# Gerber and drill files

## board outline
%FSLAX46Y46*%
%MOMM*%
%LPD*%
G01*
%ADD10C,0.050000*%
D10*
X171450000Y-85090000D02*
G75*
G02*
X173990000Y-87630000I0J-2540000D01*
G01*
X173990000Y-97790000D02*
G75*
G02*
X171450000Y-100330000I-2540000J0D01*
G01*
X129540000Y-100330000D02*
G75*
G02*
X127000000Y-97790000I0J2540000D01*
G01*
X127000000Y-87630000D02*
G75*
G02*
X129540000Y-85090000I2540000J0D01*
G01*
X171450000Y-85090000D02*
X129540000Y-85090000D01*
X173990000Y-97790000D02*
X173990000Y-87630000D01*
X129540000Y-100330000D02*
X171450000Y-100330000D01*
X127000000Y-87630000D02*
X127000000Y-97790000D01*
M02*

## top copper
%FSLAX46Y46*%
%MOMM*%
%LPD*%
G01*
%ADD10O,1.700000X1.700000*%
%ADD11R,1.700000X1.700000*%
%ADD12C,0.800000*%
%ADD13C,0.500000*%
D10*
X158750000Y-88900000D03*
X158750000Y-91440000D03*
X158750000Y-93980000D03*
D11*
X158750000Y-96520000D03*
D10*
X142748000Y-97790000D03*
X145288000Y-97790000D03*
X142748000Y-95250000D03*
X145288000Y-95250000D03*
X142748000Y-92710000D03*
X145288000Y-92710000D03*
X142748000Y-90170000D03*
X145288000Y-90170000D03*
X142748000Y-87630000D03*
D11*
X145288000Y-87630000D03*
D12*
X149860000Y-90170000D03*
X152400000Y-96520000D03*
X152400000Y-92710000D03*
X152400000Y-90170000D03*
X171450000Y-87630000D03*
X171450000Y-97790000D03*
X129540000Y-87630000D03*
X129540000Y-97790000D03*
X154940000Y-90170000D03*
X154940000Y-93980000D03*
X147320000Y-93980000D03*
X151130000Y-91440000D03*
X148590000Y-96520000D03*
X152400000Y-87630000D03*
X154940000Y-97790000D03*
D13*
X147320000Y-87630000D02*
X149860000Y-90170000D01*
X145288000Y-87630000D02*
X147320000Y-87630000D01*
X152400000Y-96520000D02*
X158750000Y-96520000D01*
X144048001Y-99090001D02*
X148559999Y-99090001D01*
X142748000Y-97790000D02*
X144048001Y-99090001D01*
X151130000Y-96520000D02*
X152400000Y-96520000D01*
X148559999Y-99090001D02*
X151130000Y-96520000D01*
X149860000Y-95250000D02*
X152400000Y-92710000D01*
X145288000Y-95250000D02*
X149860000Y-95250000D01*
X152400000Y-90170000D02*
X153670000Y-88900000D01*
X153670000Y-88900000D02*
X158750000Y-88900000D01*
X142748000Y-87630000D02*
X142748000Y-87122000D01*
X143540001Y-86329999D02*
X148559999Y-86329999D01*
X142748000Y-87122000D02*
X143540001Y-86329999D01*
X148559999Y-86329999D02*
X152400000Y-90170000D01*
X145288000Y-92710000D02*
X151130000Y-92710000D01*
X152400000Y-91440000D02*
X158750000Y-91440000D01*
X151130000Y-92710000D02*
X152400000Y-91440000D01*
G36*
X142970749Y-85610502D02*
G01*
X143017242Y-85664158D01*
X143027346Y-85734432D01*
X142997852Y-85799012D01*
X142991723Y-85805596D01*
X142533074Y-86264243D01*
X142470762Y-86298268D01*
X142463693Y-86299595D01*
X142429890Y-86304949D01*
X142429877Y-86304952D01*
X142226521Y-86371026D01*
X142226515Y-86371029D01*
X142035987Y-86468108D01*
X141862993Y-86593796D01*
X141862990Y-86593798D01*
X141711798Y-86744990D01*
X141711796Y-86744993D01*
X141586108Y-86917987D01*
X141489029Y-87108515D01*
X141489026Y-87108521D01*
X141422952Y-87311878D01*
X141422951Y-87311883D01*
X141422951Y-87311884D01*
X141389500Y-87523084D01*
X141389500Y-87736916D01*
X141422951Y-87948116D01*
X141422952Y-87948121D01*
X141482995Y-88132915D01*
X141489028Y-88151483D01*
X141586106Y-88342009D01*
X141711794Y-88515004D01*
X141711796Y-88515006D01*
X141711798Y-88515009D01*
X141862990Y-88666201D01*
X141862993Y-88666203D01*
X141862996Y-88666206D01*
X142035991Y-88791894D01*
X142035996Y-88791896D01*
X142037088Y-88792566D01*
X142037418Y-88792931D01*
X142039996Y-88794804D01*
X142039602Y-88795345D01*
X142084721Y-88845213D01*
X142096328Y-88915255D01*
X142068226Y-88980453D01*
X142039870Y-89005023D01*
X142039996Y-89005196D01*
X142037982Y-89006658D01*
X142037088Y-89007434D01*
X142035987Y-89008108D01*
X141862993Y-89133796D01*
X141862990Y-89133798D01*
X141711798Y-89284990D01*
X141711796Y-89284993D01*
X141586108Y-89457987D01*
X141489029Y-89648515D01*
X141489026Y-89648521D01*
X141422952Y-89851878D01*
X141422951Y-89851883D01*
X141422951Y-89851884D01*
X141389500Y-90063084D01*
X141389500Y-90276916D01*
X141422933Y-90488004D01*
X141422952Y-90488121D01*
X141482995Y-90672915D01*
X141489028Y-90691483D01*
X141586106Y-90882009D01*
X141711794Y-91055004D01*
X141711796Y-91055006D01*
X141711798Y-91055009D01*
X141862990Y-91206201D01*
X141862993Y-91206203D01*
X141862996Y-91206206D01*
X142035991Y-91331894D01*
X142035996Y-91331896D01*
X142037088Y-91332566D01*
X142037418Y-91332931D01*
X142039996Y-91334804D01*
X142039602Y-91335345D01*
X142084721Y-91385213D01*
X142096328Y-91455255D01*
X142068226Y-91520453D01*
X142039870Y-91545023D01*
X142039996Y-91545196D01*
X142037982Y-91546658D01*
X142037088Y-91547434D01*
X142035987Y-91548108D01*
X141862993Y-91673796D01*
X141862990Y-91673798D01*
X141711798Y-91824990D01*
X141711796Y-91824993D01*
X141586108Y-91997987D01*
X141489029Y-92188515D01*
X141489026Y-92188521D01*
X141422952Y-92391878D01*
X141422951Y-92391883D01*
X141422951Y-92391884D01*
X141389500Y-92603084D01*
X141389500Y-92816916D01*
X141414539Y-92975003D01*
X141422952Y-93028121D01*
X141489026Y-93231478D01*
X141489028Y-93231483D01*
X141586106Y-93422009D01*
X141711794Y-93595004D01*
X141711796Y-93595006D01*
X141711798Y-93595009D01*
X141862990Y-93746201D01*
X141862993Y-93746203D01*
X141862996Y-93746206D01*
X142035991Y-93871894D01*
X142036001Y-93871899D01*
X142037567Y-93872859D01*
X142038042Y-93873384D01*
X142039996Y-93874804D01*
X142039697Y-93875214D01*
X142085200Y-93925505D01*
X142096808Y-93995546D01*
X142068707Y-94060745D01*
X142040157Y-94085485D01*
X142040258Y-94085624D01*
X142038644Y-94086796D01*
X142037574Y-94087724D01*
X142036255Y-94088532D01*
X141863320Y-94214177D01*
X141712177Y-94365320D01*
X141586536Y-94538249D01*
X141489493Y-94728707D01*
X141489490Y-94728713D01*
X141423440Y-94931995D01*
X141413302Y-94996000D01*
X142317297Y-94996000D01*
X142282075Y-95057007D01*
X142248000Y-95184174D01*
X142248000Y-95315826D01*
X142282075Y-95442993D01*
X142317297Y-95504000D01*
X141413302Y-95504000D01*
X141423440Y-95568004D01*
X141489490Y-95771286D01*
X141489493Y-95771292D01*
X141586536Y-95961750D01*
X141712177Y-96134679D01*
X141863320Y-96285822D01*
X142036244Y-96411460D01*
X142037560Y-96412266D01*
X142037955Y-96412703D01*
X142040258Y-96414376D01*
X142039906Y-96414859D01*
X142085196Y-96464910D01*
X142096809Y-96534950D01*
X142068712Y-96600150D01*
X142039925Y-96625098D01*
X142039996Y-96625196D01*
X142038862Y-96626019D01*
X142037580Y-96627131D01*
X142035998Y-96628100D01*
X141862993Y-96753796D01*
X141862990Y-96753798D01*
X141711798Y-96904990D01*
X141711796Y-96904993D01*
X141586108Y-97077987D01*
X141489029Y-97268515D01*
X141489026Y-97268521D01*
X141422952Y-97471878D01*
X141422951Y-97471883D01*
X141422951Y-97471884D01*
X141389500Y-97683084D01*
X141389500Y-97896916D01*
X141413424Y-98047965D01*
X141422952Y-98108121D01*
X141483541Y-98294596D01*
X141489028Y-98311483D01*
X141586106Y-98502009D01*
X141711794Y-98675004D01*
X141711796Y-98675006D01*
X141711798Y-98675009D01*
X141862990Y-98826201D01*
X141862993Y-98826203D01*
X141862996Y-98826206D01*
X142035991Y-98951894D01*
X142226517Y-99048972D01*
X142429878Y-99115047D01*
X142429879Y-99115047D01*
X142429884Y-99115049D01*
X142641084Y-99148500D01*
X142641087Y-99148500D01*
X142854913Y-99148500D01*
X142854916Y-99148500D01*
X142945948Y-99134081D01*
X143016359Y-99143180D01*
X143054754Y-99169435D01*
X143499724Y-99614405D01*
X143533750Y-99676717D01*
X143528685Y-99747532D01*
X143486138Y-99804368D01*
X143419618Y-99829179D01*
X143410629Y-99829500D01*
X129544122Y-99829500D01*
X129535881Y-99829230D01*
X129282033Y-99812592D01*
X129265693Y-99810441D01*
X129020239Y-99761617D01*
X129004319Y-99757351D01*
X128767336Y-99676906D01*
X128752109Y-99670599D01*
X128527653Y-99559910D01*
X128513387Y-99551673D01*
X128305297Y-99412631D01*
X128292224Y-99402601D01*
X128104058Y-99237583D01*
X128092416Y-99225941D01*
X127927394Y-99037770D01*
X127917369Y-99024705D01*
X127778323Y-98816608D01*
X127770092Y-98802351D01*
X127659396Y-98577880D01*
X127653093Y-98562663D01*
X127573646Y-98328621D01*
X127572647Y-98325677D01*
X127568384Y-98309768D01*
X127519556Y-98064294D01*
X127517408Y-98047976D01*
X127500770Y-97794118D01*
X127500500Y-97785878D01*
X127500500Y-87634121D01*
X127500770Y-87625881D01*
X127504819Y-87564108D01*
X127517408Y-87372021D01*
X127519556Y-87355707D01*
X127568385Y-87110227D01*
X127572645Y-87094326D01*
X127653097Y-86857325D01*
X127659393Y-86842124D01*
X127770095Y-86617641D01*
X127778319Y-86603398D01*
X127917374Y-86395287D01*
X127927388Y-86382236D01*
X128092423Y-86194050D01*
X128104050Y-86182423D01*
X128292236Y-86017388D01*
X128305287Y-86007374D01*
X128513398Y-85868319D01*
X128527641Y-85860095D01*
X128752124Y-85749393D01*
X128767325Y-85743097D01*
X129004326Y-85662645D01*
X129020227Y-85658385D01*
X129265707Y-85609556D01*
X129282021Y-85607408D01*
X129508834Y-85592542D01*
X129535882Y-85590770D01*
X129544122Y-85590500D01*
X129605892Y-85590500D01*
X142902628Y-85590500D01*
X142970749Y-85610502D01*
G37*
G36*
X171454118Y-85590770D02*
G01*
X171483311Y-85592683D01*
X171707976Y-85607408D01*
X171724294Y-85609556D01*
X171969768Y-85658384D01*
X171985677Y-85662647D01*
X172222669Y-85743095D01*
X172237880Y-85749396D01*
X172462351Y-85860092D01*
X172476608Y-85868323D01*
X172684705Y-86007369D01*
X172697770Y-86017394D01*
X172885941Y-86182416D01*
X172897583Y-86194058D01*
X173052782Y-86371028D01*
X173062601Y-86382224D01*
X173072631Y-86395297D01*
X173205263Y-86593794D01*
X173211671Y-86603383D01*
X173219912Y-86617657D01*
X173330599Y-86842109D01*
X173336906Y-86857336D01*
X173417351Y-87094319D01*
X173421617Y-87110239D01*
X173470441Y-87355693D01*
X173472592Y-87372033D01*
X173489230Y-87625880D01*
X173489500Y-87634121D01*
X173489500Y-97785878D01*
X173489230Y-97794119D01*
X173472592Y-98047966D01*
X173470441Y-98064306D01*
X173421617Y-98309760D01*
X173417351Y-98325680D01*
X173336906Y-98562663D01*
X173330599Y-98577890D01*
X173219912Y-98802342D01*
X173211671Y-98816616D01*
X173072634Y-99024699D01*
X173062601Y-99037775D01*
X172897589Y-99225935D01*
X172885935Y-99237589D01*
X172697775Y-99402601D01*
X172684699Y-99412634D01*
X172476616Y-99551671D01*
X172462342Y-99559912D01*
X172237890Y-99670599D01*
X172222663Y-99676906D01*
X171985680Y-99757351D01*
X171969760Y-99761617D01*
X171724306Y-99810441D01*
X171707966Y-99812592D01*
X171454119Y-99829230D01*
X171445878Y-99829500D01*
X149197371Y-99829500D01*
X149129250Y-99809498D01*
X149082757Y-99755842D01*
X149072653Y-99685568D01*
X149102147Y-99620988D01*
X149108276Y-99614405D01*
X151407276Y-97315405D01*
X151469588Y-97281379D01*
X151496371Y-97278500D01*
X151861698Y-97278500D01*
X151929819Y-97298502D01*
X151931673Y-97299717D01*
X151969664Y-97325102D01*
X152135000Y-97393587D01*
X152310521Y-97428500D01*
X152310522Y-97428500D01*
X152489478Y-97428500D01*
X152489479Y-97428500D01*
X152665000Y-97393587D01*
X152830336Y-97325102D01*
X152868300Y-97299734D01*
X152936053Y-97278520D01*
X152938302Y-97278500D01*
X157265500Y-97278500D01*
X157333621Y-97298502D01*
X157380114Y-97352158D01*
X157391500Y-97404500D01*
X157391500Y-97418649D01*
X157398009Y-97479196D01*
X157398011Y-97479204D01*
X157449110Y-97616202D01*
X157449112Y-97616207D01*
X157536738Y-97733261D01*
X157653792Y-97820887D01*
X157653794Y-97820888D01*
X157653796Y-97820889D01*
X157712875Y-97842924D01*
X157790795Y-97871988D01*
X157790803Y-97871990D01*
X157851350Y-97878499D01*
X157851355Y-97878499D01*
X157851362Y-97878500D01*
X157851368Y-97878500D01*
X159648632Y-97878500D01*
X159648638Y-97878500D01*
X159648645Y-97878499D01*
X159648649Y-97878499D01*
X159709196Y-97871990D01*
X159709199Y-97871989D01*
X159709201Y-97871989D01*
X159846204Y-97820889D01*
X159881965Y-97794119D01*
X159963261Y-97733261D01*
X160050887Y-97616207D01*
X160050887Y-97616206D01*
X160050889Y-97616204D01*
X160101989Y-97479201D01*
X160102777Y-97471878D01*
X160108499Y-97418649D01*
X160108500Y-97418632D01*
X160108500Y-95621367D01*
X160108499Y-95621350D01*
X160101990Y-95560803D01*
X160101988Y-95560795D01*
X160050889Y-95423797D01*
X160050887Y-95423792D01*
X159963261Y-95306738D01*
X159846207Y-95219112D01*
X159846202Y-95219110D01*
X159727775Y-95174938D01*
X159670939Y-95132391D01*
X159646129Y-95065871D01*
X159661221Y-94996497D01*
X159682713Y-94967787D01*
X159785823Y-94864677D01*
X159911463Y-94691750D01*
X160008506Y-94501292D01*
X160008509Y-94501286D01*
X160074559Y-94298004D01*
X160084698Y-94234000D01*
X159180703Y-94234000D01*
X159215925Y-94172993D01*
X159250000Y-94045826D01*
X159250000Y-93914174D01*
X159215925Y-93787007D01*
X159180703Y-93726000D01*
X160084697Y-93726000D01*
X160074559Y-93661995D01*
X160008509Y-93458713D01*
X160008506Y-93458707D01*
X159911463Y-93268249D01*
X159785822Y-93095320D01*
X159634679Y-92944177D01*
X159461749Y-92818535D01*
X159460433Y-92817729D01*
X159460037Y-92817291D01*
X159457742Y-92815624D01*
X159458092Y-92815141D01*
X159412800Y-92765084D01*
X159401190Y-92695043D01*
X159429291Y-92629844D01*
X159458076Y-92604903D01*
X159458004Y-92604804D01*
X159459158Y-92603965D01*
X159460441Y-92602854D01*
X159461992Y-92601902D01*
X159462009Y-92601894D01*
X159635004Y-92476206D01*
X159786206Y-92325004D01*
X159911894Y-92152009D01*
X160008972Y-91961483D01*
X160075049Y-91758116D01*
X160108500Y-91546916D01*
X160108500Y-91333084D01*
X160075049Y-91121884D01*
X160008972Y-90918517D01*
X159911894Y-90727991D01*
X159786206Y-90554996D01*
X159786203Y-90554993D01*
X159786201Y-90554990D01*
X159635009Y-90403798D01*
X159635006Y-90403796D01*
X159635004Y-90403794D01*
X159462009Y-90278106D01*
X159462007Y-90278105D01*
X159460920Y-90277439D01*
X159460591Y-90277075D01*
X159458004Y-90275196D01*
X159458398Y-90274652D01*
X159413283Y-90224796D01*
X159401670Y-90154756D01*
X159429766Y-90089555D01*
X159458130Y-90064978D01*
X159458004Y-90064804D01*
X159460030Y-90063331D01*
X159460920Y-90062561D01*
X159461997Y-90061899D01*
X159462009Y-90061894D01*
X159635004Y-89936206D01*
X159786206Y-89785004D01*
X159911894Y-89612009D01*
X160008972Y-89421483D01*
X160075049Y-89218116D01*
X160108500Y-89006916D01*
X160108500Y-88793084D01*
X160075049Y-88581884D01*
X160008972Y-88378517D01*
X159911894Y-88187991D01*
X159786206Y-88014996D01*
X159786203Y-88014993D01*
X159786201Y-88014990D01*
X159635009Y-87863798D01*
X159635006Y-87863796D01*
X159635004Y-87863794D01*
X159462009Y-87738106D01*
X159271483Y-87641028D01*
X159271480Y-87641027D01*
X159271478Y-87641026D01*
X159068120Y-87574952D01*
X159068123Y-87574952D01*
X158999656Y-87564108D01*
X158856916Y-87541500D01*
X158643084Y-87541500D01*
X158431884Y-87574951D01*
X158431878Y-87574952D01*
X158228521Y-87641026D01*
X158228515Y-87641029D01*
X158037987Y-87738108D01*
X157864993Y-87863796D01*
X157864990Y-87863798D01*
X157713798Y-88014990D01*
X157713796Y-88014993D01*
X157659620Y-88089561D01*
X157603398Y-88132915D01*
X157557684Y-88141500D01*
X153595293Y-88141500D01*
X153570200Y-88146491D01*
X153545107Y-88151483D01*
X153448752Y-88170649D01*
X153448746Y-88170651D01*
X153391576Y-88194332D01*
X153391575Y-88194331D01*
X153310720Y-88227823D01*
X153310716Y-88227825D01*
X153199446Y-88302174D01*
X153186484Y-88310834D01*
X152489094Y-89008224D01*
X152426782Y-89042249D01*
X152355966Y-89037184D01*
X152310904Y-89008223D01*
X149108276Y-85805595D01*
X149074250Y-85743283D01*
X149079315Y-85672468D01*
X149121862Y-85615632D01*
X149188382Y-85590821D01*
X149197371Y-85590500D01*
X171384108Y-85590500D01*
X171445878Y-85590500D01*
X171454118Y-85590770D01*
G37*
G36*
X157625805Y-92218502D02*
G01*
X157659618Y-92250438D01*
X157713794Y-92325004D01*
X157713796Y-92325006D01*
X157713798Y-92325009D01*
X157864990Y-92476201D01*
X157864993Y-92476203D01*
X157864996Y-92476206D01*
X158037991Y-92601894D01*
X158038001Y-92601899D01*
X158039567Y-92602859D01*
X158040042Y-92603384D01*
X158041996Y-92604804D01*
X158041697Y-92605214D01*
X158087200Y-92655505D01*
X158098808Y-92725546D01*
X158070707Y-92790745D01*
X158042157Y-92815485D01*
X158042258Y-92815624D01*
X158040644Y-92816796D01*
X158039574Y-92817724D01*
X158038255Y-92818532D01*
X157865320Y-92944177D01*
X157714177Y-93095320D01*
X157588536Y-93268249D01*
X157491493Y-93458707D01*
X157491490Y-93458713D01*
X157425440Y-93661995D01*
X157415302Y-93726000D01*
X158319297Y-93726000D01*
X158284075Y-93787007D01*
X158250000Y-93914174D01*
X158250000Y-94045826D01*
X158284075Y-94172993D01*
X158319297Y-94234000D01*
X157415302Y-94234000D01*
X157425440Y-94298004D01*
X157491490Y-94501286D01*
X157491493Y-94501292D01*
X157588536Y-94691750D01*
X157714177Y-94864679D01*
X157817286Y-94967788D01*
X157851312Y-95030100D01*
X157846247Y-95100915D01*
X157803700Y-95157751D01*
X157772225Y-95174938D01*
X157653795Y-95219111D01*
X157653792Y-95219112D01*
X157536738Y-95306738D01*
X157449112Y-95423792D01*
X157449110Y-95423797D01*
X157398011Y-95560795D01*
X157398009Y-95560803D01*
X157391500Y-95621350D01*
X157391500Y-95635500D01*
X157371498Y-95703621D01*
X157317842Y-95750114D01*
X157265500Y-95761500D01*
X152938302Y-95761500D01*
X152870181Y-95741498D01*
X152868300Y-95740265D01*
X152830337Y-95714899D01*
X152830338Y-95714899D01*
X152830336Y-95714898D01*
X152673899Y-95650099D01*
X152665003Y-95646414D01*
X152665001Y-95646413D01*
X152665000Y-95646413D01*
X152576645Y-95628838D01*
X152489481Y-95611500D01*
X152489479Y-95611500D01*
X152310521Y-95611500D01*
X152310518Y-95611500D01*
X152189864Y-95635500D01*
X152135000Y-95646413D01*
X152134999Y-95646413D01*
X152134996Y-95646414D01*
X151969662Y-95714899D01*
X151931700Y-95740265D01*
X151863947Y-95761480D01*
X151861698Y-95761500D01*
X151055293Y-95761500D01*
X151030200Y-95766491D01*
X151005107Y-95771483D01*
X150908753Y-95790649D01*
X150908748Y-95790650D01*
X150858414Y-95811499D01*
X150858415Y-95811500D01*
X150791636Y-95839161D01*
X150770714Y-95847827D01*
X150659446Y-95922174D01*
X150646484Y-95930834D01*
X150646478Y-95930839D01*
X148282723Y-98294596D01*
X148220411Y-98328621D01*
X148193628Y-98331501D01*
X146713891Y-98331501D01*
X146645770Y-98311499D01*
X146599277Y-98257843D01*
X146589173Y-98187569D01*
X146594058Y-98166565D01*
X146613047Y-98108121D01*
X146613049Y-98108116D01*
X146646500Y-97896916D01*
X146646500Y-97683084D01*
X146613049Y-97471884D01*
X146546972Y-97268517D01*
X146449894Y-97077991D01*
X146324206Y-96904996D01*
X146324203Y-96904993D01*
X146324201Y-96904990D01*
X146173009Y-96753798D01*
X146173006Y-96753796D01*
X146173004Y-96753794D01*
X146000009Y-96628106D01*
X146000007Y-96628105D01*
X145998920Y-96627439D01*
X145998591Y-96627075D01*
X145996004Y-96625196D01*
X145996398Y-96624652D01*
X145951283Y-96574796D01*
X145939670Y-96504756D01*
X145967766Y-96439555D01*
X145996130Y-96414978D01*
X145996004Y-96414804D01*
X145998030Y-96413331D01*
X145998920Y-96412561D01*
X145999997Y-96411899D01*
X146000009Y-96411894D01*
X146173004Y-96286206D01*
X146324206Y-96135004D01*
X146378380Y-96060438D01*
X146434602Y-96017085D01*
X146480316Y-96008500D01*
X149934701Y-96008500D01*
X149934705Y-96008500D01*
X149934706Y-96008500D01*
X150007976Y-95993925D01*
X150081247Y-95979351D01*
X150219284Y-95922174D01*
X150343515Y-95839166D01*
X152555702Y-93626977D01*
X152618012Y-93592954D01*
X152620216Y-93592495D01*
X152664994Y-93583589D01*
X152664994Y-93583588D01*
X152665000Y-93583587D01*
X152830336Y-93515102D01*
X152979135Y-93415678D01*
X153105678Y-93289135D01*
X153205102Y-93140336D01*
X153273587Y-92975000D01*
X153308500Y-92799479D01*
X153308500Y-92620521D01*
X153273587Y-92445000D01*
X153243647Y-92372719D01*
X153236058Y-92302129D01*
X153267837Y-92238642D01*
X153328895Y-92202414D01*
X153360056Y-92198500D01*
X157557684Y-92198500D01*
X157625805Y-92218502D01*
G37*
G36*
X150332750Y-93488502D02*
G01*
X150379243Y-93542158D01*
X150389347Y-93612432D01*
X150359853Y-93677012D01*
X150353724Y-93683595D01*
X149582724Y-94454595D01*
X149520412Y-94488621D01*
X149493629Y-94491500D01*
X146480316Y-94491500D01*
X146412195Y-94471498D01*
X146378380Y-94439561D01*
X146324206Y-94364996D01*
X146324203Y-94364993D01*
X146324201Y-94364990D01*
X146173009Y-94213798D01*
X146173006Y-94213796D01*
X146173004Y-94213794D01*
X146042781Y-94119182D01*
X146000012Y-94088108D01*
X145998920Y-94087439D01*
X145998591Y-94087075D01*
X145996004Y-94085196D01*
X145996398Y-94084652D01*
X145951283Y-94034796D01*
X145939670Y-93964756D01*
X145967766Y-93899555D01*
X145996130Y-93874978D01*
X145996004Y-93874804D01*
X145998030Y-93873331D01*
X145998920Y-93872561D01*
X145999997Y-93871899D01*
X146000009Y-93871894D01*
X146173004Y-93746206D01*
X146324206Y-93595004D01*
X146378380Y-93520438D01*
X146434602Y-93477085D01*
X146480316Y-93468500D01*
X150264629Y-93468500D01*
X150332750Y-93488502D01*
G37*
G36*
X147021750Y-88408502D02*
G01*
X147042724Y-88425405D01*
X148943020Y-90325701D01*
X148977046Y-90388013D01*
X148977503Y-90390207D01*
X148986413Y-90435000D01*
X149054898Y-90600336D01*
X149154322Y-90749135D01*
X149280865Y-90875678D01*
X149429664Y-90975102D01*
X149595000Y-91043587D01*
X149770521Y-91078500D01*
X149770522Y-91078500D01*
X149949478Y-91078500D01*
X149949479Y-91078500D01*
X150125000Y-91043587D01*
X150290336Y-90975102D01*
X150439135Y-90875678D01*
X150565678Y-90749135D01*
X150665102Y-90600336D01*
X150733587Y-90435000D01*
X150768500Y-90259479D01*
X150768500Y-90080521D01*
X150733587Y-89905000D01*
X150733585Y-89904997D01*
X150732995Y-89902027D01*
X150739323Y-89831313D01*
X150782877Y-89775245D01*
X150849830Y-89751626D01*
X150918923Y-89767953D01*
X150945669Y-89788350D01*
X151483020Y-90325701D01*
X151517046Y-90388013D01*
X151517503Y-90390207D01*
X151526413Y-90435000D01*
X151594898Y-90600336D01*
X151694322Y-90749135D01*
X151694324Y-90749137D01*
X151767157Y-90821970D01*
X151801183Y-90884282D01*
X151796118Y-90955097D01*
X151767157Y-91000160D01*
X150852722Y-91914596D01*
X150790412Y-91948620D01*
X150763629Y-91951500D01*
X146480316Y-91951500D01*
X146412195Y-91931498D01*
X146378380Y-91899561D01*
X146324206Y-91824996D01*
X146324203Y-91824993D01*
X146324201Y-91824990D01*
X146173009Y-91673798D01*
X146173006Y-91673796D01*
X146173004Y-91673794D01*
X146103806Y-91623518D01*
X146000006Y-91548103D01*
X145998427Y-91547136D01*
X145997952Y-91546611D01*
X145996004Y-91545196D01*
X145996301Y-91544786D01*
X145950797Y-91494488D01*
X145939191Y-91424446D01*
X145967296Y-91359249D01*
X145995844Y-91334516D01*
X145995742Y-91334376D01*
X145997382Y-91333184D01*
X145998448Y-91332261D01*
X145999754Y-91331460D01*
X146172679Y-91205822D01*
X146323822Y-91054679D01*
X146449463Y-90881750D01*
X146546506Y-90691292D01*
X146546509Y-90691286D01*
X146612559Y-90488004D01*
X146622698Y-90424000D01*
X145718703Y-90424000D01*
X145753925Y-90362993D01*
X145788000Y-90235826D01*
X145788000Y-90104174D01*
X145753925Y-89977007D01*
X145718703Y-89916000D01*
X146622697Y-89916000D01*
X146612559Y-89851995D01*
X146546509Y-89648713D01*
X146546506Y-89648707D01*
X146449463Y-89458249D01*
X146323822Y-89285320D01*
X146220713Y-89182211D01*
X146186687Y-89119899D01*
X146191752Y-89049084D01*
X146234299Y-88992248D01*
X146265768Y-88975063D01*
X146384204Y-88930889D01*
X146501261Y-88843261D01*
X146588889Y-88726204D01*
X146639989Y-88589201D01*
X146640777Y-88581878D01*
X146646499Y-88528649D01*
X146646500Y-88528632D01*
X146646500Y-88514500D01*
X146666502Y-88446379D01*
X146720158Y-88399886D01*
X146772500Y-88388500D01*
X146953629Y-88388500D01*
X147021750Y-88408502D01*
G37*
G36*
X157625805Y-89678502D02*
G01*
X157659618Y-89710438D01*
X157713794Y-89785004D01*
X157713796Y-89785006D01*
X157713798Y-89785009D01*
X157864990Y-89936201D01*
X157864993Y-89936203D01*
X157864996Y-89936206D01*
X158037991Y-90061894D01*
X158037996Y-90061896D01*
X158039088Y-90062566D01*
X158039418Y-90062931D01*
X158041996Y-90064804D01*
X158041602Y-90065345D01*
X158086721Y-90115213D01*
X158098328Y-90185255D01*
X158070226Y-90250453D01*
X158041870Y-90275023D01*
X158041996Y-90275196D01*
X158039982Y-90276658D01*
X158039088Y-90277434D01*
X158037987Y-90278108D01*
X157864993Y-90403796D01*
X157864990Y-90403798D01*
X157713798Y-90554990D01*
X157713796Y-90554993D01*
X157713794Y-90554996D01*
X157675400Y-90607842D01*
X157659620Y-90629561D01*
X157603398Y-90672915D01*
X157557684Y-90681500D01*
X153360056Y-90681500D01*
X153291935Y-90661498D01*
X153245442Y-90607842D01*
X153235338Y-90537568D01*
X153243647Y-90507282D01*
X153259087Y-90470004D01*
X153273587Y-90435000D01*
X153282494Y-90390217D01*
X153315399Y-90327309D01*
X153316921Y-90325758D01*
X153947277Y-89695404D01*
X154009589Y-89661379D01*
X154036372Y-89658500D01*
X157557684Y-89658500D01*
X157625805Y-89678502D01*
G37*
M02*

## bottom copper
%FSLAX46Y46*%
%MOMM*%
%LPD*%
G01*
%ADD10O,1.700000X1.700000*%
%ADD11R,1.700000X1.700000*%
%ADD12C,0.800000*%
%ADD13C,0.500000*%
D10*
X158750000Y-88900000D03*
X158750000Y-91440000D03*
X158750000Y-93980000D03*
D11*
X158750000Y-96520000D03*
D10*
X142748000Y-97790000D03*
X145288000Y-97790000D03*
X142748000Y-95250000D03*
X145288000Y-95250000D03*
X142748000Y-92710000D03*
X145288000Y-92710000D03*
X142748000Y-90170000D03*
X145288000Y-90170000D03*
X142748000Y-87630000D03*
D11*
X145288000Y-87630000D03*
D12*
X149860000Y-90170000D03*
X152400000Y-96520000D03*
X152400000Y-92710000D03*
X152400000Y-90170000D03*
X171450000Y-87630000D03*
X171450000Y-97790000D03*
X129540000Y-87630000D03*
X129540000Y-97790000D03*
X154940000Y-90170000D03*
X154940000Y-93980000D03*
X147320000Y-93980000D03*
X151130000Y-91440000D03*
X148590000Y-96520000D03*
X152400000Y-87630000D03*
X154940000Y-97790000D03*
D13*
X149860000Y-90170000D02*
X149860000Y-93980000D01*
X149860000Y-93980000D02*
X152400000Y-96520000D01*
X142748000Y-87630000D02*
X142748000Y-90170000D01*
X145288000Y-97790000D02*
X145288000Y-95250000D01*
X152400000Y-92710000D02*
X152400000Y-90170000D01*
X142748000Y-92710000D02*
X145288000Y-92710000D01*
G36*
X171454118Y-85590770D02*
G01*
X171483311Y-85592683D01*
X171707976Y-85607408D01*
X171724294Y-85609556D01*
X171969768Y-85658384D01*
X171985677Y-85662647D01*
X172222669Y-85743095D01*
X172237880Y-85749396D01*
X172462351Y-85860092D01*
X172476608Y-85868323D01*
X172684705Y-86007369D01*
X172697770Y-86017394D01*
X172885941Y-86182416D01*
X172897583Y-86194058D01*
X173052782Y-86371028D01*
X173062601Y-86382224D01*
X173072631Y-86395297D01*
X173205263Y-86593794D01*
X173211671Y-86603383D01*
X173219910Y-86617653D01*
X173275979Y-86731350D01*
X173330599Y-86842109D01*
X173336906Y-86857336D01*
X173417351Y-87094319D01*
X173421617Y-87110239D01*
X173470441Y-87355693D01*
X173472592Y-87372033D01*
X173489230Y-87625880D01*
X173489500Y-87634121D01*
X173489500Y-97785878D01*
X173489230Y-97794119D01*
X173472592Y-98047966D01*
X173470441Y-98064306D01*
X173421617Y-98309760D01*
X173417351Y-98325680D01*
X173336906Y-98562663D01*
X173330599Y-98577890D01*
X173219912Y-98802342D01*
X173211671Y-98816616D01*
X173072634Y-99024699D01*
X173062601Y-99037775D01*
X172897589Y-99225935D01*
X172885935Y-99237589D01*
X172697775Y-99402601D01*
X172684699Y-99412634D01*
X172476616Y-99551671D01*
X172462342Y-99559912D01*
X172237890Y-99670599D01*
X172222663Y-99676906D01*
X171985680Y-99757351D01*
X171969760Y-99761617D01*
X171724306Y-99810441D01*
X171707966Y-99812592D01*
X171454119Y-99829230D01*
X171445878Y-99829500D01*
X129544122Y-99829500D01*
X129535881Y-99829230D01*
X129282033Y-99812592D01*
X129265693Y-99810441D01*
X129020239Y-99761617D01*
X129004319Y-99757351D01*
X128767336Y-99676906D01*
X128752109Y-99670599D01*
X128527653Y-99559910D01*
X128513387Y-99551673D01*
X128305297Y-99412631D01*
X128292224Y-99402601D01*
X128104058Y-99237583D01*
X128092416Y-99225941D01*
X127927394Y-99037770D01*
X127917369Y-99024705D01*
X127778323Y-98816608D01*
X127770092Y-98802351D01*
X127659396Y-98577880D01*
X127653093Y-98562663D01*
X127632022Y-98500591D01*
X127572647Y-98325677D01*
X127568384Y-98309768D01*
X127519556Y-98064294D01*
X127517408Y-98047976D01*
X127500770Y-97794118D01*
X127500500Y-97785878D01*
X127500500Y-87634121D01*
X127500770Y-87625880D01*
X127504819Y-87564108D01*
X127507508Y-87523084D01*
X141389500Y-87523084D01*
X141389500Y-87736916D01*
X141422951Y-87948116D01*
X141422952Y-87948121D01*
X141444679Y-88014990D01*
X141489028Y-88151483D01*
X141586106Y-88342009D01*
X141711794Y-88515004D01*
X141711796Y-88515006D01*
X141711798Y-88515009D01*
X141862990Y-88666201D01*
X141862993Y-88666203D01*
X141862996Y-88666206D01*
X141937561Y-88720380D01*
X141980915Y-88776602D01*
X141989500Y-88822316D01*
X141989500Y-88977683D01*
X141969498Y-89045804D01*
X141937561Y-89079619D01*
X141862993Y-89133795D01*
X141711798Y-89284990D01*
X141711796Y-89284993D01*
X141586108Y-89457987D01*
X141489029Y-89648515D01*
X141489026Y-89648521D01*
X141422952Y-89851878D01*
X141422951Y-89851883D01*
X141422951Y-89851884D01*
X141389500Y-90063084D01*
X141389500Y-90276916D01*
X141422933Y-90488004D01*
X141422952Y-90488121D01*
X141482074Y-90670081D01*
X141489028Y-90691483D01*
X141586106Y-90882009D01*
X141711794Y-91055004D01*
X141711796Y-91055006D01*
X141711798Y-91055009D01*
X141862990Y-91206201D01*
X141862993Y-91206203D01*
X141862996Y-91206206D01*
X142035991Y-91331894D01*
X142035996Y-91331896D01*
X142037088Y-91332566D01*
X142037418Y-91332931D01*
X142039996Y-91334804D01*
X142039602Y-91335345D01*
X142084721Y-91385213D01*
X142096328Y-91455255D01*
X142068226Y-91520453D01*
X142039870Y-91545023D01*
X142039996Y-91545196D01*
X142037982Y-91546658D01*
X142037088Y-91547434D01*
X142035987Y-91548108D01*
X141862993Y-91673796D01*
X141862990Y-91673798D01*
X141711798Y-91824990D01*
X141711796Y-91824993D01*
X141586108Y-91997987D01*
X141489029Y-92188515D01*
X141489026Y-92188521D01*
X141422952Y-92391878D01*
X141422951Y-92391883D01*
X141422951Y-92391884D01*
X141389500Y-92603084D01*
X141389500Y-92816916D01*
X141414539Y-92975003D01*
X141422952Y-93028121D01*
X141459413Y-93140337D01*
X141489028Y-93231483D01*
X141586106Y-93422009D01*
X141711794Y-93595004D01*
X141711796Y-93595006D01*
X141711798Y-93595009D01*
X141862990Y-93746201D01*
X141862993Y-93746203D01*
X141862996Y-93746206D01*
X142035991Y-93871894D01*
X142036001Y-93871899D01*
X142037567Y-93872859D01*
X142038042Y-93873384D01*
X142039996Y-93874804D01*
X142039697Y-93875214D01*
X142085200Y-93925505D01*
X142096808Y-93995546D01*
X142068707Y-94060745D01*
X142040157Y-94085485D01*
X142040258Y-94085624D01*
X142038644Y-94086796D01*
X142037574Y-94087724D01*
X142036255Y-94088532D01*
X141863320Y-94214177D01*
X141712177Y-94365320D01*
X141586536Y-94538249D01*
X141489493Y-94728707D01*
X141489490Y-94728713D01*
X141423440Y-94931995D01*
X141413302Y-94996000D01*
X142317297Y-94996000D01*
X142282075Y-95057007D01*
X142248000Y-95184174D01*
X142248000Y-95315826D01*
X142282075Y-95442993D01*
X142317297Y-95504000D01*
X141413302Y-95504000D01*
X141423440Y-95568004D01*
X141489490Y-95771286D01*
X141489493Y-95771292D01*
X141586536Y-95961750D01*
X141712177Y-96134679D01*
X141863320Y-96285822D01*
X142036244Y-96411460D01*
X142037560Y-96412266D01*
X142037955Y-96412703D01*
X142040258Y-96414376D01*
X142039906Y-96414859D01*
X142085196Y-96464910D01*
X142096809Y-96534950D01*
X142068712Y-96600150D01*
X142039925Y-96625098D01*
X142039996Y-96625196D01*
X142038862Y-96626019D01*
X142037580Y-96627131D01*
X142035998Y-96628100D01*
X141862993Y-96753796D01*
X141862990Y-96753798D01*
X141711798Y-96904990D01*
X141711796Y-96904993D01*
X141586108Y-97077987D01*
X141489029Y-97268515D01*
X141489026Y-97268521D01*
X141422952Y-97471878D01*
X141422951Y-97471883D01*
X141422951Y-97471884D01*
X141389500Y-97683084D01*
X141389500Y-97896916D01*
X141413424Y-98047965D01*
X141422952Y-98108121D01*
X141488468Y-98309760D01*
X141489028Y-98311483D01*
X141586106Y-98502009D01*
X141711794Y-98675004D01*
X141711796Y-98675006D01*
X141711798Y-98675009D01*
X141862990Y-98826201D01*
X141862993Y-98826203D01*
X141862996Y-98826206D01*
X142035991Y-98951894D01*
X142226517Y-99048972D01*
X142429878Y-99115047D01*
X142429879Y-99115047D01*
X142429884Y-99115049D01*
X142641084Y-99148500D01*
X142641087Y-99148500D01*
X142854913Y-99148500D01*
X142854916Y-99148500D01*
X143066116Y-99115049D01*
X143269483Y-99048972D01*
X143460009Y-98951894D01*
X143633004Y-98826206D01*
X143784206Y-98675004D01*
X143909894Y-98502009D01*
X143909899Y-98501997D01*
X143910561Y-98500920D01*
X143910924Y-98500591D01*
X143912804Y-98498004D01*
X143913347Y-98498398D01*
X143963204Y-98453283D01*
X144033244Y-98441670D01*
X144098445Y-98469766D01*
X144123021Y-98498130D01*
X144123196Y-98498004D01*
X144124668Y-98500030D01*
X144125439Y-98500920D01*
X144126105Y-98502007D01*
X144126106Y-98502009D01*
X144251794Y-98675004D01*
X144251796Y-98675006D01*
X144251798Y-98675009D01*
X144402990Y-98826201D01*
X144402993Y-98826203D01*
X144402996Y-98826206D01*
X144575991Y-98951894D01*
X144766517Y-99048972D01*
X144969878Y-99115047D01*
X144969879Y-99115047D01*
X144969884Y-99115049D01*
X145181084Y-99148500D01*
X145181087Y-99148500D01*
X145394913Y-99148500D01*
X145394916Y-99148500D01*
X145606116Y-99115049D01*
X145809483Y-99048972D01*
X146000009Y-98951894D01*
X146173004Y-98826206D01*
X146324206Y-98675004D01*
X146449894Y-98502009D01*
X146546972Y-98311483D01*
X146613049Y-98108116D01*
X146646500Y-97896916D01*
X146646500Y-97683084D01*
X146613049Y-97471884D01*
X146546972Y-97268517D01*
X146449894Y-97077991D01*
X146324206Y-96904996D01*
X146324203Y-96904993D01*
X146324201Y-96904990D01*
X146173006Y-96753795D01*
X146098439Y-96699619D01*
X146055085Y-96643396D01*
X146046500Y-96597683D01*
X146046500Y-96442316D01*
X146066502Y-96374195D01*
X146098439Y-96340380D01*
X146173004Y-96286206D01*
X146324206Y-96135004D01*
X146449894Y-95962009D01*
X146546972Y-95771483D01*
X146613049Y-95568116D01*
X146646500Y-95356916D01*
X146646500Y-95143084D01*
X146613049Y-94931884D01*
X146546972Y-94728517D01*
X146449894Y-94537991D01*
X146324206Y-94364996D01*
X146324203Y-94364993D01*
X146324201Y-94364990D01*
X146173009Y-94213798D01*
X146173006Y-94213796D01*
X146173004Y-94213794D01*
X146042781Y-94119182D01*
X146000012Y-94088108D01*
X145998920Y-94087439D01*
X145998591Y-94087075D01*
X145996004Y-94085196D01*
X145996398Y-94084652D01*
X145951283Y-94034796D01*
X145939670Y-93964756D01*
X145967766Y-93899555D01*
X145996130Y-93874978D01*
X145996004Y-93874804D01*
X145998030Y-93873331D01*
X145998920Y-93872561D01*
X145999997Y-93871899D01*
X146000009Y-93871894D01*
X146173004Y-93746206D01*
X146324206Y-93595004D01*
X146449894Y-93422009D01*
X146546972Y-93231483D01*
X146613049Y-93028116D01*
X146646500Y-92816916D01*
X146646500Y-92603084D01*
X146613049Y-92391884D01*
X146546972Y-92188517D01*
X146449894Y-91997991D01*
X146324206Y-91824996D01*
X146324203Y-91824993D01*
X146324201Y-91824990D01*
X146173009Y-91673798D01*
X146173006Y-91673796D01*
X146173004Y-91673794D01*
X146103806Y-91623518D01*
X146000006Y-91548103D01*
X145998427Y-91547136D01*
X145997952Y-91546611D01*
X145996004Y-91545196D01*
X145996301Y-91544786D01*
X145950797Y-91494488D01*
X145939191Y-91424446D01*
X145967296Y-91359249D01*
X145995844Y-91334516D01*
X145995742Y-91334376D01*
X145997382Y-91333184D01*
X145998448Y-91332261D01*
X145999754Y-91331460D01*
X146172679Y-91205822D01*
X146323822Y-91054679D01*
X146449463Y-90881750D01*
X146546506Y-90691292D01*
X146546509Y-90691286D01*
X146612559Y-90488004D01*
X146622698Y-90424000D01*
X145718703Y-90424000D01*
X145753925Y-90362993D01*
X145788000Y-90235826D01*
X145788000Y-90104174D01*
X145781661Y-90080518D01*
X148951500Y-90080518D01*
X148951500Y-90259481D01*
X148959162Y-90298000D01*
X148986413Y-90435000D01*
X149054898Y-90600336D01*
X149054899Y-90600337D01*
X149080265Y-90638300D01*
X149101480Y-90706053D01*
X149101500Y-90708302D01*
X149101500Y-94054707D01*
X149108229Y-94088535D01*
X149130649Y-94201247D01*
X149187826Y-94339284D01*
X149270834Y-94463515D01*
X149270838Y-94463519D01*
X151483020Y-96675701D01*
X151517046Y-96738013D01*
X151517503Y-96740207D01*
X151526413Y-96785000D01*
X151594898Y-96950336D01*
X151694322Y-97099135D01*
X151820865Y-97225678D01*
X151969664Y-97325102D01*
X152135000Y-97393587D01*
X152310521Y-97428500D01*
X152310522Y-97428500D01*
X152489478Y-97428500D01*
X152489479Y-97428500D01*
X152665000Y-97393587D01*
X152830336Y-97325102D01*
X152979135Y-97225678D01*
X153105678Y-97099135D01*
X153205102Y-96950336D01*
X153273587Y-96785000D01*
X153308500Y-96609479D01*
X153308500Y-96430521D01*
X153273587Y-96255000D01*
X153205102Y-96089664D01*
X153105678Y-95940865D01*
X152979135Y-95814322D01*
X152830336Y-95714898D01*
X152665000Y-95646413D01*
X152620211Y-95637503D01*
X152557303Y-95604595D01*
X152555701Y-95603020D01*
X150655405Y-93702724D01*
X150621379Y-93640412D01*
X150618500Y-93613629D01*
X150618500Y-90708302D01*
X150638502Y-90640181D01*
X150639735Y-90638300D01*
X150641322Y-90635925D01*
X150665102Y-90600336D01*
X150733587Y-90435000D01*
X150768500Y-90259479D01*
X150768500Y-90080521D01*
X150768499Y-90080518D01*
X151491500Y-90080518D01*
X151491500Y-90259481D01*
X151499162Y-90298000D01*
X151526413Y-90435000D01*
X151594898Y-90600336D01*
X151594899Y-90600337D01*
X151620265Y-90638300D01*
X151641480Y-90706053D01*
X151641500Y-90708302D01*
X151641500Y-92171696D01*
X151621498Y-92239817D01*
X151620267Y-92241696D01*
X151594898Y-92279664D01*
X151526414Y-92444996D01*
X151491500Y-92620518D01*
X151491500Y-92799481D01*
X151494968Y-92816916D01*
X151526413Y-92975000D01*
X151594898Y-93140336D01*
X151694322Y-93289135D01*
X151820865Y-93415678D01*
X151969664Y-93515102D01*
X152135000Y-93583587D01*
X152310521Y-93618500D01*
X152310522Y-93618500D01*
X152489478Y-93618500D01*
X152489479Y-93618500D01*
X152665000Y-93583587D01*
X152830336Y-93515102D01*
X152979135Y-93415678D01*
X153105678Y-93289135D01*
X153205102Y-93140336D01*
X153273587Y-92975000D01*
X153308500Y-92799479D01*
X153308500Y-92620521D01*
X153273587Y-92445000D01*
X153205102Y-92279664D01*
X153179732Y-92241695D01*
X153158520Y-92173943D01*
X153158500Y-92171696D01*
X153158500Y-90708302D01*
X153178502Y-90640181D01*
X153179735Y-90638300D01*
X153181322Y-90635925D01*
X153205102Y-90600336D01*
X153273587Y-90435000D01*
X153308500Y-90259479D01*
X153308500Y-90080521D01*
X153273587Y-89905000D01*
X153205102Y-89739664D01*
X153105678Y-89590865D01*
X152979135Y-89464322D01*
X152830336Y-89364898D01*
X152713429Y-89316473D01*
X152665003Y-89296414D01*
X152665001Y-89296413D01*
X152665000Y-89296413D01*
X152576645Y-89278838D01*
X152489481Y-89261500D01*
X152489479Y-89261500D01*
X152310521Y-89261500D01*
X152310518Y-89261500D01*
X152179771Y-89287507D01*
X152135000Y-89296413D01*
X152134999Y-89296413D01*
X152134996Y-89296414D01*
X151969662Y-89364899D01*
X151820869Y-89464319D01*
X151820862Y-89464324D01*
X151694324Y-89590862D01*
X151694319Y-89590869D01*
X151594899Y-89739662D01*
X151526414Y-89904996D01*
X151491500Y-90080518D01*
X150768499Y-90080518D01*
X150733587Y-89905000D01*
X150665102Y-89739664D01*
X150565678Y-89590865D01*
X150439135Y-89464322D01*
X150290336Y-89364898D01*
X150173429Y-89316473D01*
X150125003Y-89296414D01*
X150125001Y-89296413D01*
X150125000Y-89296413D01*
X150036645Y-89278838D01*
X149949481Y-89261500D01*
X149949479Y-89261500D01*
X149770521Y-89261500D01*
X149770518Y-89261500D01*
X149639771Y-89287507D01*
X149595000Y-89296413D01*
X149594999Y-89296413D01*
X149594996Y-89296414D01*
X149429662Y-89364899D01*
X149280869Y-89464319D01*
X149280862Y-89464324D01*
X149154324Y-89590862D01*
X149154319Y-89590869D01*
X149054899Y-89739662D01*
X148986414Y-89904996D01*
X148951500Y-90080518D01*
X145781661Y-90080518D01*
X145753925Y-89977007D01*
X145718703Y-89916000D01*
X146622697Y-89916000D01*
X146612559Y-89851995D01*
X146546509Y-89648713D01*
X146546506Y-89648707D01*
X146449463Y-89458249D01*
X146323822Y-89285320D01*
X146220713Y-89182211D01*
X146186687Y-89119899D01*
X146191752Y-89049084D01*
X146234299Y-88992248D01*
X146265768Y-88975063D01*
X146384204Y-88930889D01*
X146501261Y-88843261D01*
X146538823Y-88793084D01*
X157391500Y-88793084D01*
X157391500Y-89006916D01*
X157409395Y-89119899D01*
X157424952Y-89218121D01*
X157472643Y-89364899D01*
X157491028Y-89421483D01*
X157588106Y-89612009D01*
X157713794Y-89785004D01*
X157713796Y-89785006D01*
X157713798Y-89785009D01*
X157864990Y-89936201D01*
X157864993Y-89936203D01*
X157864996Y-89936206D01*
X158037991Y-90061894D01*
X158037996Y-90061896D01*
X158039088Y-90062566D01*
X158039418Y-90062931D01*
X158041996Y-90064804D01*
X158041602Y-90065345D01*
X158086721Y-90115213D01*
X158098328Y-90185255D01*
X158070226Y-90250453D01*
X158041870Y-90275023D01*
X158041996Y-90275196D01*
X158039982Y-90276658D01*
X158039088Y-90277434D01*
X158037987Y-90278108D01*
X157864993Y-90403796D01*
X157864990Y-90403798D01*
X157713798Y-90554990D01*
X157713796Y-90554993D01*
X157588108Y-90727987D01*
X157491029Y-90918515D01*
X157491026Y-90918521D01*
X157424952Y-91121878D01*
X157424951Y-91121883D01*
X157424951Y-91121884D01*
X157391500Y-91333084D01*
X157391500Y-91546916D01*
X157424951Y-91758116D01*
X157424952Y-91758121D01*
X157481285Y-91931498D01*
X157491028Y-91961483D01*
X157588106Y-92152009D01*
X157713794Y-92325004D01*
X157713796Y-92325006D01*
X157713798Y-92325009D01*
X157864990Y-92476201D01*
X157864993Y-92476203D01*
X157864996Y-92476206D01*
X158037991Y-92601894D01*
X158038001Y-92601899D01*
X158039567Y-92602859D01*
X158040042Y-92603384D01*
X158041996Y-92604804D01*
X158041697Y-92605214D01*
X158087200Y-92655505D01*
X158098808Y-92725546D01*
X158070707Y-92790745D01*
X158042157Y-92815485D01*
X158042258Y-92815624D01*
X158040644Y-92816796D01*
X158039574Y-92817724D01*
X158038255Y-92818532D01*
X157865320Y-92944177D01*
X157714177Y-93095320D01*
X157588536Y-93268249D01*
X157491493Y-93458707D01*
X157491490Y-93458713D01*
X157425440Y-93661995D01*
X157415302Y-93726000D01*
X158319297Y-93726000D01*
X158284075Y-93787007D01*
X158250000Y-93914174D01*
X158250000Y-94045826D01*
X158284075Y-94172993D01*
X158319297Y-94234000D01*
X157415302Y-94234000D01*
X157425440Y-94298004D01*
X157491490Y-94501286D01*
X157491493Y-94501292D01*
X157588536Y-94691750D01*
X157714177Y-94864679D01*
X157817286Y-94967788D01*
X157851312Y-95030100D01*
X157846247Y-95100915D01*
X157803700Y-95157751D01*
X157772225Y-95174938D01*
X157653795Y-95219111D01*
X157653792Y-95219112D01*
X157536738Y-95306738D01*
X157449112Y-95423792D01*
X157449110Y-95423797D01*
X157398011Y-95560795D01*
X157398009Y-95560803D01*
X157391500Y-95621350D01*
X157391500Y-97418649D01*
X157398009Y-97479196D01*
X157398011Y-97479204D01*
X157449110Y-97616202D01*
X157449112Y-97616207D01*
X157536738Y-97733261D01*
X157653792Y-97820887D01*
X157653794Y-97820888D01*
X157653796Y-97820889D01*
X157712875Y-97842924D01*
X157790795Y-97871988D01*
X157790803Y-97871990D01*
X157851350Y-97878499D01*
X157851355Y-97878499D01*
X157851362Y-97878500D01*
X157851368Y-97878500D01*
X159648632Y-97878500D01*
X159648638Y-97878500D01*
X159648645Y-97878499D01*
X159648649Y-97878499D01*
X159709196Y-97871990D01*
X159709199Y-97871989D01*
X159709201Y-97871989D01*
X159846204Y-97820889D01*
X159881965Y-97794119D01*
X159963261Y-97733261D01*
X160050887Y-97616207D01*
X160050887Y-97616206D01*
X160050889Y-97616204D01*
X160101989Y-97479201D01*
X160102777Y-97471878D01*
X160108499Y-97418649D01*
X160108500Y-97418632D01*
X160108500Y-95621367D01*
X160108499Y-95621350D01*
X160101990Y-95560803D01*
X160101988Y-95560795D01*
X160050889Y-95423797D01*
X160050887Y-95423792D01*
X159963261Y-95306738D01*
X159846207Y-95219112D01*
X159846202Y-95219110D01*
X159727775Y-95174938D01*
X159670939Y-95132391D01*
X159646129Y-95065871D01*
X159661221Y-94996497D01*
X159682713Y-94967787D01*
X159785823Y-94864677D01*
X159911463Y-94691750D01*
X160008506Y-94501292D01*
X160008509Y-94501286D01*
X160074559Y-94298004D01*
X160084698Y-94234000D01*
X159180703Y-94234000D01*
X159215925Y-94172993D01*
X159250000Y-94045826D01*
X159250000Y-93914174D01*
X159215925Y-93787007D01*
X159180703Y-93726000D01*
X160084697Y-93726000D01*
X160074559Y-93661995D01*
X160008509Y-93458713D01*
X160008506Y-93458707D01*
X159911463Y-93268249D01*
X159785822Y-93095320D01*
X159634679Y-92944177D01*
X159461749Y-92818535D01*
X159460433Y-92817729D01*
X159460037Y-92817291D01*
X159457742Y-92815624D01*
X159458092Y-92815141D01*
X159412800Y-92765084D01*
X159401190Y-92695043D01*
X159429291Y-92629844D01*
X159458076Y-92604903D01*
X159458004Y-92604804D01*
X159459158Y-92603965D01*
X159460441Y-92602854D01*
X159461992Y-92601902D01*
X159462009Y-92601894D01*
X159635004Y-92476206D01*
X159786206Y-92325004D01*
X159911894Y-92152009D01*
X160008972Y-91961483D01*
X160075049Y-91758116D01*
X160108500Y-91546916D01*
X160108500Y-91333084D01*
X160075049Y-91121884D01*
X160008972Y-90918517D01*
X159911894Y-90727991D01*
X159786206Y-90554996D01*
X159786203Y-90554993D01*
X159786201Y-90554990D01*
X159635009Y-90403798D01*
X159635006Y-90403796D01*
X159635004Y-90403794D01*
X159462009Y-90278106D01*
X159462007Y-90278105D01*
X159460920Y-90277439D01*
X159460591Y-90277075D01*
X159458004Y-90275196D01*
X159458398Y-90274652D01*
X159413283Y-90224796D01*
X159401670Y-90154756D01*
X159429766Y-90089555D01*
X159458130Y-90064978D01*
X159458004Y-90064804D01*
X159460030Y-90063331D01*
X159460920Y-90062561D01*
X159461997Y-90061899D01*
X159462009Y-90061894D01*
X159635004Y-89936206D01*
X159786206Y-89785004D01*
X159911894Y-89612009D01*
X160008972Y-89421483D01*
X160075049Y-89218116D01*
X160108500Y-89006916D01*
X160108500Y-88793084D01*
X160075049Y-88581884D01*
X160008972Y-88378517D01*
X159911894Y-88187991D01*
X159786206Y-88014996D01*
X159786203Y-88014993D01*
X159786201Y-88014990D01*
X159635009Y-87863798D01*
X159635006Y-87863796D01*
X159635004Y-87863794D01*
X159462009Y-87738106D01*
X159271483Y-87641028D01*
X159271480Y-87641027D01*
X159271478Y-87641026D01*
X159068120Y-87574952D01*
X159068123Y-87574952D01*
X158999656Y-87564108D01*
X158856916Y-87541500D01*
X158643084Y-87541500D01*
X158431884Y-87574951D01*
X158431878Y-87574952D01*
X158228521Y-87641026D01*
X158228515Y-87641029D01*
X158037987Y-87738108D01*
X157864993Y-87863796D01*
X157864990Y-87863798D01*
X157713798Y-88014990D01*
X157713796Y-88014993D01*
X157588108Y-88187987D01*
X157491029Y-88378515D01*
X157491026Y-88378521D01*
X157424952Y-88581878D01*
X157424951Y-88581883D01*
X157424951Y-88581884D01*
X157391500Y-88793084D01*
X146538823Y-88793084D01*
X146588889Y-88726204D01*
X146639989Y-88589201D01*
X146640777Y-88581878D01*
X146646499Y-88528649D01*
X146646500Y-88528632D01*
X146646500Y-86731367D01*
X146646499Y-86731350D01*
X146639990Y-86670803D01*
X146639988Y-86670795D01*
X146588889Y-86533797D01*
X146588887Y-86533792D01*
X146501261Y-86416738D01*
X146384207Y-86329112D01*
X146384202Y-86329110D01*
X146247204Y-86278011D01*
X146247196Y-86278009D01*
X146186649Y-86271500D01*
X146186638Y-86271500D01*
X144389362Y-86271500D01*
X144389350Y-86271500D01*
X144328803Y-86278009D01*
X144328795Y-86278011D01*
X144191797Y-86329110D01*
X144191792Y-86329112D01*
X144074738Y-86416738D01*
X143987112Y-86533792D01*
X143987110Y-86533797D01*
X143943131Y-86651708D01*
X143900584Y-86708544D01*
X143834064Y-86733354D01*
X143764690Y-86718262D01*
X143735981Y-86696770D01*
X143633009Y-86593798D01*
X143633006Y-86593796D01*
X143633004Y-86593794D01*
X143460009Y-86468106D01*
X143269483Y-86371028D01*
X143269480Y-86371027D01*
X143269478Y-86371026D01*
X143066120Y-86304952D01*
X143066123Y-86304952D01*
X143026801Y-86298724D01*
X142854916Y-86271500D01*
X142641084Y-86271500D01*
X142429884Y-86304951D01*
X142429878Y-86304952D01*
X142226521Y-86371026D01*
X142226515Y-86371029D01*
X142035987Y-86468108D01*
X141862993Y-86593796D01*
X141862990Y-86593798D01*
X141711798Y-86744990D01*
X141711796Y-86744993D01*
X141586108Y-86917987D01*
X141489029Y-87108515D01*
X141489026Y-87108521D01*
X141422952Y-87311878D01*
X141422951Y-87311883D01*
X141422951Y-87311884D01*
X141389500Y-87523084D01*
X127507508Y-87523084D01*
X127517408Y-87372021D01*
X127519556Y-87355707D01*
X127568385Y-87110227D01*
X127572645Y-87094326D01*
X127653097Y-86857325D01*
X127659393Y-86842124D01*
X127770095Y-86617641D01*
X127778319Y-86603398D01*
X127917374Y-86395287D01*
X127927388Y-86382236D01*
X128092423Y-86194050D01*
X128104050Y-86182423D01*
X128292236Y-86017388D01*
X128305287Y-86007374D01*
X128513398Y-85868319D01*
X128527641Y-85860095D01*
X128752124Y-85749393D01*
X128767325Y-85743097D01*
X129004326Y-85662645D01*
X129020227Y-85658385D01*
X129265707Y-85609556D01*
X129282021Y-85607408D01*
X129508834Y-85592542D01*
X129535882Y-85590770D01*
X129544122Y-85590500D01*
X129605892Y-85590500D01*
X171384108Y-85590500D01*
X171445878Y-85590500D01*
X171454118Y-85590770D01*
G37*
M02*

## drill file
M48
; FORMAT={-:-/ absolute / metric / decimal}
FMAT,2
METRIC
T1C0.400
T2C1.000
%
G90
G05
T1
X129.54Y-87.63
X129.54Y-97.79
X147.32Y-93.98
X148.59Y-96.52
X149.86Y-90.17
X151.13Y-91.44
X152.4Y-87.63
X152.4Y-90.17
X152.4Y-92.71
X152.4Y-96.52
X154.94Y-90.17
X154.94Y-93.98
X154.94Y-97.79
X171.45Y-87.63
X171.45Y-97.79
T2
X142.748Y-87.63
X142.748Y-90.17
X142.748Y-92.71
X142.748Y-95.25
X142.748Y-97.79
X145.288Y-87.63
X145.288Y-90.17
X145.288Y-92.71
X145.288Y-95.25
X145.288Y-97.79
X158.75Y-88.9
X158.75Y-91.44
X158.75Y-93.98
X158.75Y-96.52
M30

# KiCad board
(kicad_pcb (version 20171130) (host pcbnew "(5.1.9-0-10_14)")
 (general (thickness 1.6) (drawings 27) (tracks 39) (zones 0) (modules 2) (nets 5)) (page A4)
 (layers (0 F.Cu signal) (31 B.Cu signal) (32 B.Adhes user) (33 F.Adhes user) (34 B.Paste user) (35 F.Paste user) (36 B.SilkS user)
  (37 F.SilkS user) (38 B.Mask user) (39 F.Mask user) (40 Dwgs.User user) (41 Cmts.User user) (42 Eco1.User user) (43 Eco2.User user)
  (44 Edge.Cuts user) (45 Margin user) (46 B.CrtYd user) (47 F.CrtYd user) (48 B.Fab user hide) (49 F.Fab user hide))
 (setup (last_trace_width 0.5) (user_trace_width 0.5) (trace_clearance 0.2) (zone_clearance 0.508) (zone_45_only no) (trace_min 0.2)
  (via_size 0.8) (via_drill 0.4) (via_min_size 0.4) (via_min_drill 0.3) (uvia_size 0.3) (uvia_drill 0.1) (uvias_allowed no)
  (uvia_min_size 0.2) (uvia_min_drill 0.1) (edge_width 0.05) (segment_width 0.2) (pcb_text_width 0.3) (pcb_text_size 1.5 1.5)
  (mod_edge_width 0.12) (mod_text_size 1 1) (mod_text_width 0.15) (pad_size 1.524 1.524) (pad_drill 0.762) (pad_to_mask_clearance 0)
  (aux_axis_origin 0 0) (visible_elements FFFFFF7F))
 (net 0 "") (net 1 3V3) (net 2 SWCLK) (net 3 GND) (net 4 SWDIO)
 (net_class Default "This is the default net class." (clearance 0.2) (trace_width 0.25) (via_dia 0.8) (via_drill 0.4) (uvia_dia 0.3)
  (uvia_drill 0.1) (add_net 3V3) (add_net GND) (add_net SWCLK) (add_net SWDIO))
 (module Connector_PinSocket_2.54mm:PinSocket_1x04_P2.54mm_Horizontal (layer F.Cu) (at 158.75 96.52 180)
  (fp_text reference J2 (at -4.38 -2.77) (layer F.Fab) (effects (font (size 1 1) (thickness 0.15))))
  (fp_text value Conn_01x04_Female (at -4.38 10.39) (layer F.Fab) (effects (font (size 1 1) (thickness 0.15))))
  (pad 4 thru_hole oval (at 0 7.62 180) (size 1.7 1.7) (drill 1) (layers *.Cu *.Mask) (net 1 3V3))
  (pad 3 thru_hole oval (at 0 5.08 180) (size 1.7 1.7) (drill 1) (layers *.Cu *.Mask) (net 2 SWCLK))
  (pad 2 thru_hole oval (at 0 2.54 180) (size 1.7 1.7) (drill 1) (layers *.Cu *.Mask) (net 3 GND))
  (pad 1 thru_hole rect (at 0 0 180) (size 1.7 1.7) (drill 1) (layers *.Cu *.Mask) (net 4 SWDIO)))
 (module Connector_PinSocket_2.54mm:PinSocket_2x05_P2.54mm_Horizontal (layer F.Cu) (at 145.288 87.63)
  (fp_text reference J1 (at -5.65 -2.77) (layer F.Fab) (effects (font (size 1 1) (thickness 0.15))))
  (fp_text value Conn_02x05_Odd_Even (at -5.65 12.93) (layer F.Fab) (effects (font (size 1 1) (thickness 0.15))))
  (pad 10 thru_hole oval (at -2.54 10.16) (size 1.7 1.7) (drill 1) (layers *.Cu *.Mask) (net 4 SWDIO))
  (pad 9 thru_hole oval (at 0 10.16) (size 1.7 1.7) (drill 1) (layers *.Cu *.Mask) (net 1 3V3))
  (pad 8 thru_hole oval (at -2.54 7.62) (size 1.7 1.7) (drill 1) (layers *.Cu *.Mask) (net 3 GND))
  (pad 7 thru_hole oval (at 0 7.62) (size 1.7 1.7) (drill 1) (layers *.Cu *.Mask) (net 1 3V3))
  (pad 6 thru_hole oval (at -2.54 5.08) (size 1.7 1.7) (drill 1) (layers *.Cu *.Mask) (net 2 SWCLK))
  (pad 5 thru_hole oval (at 0 5.08) (size 1.7 1.7) (drill 1) (layers *.Cu *.Mask) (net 2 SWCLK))
  (pad 4 thru_hole oval (at -2.54 2.54) (size 1.7 1.7) (drill 1) (layers *.Cu *.Mask) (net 1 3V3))
  (pad 3 thru_hole oval (at 0 2.54) (size 1.7 1.7) (drill 1) (layers *.Cu *.Mask) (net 3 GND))
  (pad 2 thru_hole oval (at -2.54 0) (size 1.7 1.7) (drill 1) (layers *.Cu *.Mask) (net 1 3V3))
  (pad 1 thru_hole rect (at 0 0) (size 1.7 1.7) (drill 1) (layers *.Cu *.Mask) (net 4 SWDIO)))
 (gr_arc (start 171.45 87.63) (end 173.99 87.63) (angle -90) (layer Edge.Cuts) (width 0.05))
 (gr_arc (start 171.45 97.79) (end 171.45 100.33) (angle -90) (layer Edge.Cuts) (width 0.05))
 (gr_arc (start 129.54 97.79) (end 127 97.79) (angle -90) (layer Edge.Cuts) (width 0.05))
 (gr_arc (start 129.54 87.63) (end 129.54 85.09) (angle -90) (layer Edge.Cuts) (width 0.05))
 (gr_line (start 171.45 85.09) (end 129.54 85.09) (layer Edge.Cuts) (width 0.05))
 (gr_line (start 173.99 97.79) (end 173.99 87.63) (layer Edge.Cuts) (width 0.05))
 (gr_line (start 129.54 100.33) (end 171.45 100.33) (layer Edge.Cuts) (width 0.05))
 (gr_line (start 127 87.63) (end 127 97.79) (layer Edge.Cuts) (width 0.05))
 (segment (start 147.32 87.63) (end 149.86 90.17) (width 0.5) (layer F.Cu) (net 4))
 (via (at 149.86 90.17) (size 0.8) (drill 0.4) (layers F.Cu B.Cu) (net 4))
 (segment (start 145.288 87.63) (end 147.32 87.63) (width 0.5) (layer F.Cu) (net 4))
 (segment (start 149.86 90.17) (end 149.86 93.98) (width 0.5) (layer B.Cu) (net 4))
 (via (at 152.4 96.52) (size 0.8) (drill 0.4) (layers F.Cu B.Cu) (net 4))
 (segment (start 149.86 93.98) (end 152.4 96.52) (width 0.5) (layer B.Cu) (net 4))
 (segment (start 152.4 96.52) (end 158.75 96.52) (width 0.5) (layer F.Cu) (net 4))
 (segment (start 144.048001 99.090001) (end 148.559999 99.090001) (width 0.5) (layer F.Cu) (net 4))
 (segment (start 142.748 97.79) (end 144.048001 99.090001) (width 0.5) (layer F.Cu) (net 4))
 (segment (start 151.13 96.52) (end 152.4 96.52) (width 0.5) (layer F.Cu) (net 4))
 (segment (start 148.559999 99.090001) (end 151.13 96.52) (width 0.5) (layer F.Cu) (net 4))
 (segment (start 142.748 87.63) (end 142.748 90.17) (width 0.5) (layer B.Cu) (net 1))
 (segment (start 145.288 97.79) (end 145.288 95.25) (width 0.5) (layer B.Cu) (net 1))
 (segment (start 149.86 95.25) (end 152.4 92.71) (width 0.5) (layer F.Cu) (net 1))
 (via (at 152.4 92.71) (size 0.8) (drill 0.4) (layers F.Cu B.Cu) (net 1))
 (segment (start 145.288 95.25) (end 149.86 95.25) (width 0.5) (layer F.Cu) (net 1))
 (via (at 152.4 90.17) (size 0.8) (drill 0.4) (layers F.Cu B.Cu) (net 1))
 (segment (start 152.4 92.71) (end 152.4 90.17) (width 0.5) (layer B.Cu) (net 1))
 (segment (start 152.4 90.17) (end 153.67 88.9) (width 0.5) (layer F.Cu) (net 1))
 (segment (start 153.67 88.9) (end 158.75 88.9) (width 0.5) (layer F.Cu) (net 1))
 (segment (start 142.748 87.63) (end 142.748 87.122) (width 0.5) (layer F.Cu) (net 1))
 (segment (start 143.540001 86.329999) (end 148.559999 86.329999) (width 0.5) (layer F.Cu) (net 1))
 (segment (start 142.748 87.122) (end 143.540001 86.329999) (width 0.5) (layer F.Cu) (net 1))
 (segment (start 148.559999 86.329999) (end 152.4 90.17) (width 0.5) (layer F.Cu) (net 1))
 (via (at 171.45 87.63) (size 0.8) (drill 0.4) (layers F.Cu B.Cu) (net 3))
 (via (at 171.45 97.79) (size 0.8) (drill 0.4) (layers F.Cu B.Cu) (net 3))
 (via (at 129.54 87.63) (size 0.8) (drill 0.4) (layers F.Cu B.Cu) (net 3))
 (via (at 129.54 97.79) (size 0.8) (drill 0.4) (layers F.Cu B.Cu) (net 3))
 (via (at 154.94 90.17) (size 0.8) (drill 0.4) (layers F.Cu B.Cu) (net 3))
 (via (at 154.94 93.98) (size 0.8) (drill 0.4) (layers F.Cu B.Cu) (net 3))
 (via (at 147.32 93.98) (size 0.8) (drill 0.4) (layers F.Cu B.Cu) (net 3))
 (via (at 151.13 91.44) (size 0.8) (drill 0.4) (layers F.Cu B.Cu) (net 3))
 (via (at 148.59 96.52) (size 0.8) (drill 0.4) (layers F.Cu B.Cu) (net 3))
 (via (at 152.4 87.63) (size 0.8) (drill 0.4) (layers F.Cu B.Cu) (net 3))
 (via (at 154.94 97.79) (size 0.8) (drill 0.4) (layers F.Cu B.Cu) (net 3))
 (segment (start 142.748 92.71) (end 145.288 92.71) (width 0.5) (layer B.Cu) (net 2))
 (segment (start 145.288 92.71) (end 151.13 92.71) (width 0.5) (layer F.Cu) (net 2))
 (segment (start 152.4 91.44) (end 158.75 91.44) (width 0.5) (layer F.Cu) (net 2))
 (segment (start 151.13 92.71) (end 152.4 91.44) (width 0.5) (layer F.Cu) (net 2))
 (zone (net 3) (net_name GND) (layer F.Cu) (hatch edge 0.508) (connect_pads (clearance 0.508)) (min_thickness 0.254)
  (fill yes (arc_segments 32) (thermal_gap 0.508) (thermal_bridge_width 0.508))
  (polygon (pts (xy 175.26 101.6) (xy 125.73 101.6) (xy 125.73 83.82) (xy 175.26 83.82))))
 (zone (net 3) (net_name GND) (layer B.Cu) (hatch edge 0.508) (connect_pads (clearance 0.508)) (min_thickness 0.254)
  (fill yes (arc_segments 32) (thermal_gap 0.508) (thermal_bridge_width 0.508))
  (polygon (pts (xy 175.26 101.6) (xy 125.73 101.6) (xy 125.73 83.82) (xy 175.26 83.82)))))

